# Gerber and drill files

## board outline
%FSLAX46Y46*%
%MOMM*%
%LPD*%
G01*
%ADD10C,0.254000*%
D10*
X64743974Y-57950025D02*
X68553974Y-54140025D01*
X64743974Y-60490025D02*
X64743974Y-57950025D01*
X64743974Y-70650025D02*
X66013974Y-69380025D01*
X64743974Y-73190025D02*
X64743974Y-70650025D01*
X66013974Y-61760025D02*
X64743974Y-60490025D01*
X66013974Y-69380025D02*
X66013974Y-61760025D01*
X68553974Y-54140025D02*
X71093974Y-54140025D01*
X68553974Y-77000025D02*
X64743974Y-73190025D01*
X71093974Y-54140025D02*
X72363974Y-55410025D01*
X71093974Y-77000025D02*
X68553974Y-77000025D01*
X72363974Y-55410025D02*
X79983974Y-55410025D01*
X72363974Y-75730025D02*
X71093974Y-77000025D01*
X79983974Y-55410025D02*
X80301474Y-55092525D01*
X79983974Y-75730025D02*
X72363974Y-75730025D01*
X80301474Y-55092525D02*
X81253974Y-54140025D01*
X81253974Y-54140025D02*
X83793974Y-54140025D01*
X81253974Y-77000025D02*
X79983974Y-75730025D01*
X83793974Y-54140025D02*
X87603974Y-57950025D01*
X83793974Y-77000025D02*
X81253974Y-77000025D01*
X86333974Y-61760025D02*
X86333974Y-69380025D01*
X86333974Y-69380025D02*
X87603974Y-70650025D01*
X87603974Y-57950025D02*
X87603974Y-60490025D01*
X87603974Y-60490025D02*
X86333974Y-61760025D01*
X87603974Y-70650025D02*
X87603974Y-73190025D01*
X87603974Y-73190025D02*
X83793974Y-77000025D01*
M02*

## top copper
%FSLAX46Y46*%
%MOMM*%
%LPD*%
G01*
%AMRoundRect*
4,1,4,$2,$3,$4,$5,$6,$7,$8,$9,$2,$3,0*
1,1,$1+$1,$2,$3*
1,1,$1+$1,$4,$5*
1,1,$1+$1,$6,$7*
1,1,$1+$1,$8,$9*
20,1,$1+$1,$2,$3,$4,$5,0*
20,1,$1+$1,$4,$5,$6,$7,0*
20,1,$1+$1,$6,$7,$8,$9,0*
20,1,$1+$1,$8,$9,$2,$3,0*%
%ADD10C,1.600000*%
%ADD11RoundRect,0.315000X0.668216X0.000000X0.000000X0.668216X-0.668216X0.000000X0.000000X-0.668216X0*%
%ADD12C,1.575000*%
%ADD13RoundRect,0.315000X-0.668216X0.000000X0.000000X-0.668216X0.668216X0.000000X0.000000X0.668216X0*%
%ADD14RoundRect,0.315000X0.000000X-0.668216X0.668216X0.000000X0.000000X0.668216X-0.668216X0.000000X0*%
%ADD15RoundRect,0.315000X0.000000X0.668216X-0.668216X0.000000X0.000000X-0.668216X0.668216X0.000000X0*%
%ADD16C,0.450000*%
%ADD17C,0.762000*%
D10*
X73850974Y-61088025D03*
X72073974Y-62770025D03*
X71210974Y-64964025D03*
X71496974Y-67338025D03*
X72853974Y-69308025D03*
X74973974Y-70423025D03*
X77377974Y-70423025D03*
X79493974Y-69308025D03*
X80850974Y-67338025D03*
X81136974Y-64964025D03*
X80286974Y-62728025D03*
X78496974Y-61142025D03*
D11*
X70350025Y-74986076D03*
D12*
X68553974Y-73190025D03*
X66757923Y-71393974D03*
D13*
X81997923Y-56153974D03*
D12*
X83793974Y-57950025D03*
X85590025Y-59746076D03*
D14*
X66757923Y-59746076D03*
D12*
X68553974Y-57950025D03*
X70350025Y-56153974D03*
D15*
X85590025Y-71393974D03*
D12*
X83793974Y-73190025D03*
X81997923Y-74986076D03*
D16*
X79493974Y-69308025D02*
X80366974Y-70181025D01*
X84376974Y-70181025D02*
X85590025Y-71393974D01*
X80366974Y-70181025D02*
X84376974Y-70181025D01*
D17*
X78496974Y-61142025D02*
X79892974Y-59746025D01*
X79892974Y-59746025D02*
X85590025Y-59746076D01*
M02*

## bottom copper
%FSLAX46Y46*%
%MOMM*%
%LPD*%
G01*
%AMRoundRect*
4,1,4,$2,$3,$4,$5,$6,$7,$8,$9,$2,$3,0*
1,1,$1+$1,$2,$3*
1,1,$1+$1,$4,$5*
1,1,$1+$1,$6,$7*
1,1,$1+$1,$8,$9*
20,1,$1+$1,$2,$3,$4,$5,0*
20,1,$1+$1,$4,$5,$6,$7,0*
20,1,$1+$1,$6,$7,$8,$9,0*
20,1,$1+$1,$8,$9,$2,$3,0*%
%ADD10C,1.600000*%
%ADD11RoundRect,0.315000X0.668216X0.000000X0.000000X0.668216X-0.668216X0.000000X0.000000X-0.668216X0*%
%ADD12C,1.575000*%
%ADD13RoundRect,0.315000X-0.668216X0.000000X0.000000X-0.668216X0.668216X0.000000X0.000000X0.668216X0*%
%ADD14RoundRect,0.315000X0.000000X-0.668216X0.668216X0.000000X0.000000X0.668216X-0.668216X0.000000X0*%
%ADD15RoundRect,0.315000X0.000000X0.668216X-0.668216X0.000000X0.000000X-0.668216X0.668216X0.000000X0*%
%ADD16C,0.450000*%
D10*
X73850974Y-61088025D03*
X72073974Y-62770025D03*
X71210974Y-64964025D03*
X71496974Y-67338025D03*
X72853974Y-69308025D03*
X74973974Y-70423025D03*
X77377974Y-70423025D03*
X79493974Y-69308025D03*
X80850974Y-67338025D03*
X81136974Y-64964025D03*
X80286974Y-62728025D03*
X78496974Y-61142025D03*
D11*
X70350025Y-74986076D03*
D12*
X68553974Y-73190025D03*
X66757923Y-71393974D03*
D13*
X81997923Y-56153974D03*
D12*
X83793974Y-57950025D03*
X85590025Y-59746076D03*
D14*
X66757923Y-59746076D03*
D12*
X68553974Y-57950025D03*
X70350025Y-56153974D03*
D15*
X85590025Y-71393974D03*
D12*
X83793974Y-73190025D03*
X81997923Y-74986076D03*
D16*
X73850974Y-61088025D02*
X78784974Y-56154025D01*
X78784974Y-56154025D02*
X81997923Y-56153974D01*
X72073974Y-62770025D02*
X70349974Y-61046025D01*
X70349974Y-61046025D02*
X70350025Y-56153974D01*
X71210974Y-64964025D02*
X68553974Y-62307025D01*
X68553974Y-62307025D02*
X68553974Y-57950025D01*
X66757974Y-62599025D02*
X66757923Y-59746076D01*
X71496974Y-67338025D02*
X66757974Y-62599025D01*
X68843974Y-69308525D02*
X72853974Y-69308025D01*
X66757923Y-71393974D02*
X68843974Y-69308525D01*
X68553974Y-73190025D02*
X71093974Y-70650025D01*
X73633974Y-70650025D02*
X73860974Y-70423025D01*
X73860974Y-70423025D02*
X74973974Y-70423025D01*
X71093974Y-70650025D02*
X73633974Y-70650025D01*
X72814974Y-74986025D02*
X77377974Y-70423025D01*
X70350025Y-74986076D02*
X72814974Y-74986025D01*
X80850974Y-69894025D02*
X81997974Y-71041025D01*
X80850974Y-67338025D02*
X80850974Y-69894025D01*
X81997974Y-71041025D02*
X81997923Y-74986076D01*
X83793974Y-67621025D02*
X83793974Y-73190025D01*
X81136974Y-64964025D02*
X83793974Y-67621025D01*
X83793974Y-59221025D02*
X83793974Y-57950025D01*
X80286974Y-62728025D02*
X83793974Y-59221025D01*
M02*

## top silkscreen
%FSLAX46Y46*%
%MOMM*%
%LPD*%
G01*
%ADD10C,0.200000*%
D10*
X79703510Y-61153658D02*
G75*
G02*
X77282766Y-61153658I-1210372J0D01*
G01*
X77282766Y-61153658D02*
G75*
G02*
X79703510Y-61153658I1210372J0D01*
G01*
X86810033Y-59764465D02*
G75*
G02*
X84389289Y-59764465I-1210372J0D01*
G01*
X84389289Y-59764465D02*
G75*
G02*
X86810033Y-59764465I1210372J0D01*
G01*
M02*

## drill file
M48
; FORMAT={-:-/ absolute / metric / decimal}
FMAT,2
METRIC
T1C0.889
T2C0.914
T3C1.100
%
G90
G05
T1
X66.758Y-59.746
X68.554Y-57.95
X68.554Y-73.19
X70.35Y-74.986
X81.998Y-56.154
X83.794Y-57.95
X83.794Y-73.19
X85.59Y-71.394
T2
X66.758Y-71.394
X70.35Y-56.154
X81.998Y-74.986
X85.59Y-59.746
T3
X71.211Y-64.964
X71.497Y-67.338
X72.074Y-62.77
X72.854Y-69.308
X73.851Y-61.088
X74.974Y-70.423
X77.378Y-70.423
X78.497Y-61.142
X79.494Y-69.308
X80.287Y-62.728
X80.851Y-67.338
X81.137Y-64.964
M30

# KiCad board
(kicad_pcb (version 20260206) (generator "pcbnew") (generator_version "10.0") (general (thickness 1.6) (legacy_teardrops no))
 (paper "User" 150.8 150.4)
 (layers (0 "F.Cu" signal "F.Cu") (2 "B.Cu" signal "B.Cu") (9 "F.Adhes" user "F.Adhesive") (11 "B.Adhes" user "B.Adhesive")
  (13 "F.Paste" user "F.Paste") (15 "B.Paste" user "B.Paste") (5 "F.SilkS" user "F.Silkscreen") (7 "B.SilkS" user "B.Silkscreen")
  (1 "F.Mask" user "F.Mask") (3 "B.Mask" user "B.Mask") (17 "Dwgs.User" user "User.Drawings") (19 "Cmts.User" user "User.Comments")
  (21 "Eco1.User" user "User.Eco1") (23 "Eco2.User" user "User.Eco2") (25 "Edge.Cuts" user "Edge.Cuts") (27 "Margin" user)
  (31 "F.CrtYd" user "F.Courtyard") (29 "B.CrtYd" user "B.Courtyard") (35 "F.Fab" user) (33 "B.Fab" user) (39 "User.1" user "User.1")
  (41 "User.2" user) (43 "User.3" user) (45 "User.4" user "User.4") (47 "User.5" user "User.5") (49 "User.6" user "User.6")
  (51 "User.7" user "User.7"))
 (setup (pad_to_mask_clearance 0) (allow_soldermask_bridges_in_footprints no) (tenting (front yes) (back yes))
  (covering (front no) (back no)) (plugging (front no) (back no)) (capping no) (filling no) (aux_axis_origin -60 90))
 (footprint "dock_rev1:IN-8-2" (layer "F.Cu") (at 76.173974 65.570025)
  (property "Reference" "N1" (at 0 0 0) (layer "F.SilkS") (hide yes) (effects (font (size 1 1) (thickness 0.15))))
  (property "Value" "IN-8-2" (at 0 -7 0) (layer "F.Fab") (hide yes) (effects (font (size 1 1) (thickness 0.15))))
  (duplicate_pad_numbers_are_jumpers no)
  (pad "2" thru_hole circle (at -2.323 -4.482) (size 1.6 1.6) (drill 1.1) (layers "*.Cu" "*.Mask") (remove_unused_layers no) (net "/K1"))
  (pad "3" thru_hole circle (at -4.1 -2.8) (size 1.6 1.6) (drill 1.1) (layers "*.Cu" "*.Mask") (remove_unused_layers no) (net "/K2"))
  (pad "4" thru_hole circle (at -4.963 -0.606) (size 1.6 1.6) (drill 1.1) (layers "*.Cu" "*.Mask") (remove_unused_layers no) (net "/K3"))
  (pad "5" thru_hole circle (at -4.677 1.768) (size 1.6 1.6) (drill 1.1) (layers "*.Cu" "*.Mask") (remove_unused_layers no) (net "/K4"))
  (pad "6" thru_hole circle (at -3.32 3.738) (size 1.6 1.6) (drill 1.1) (layers "*.Cu" "*.Mask") (remove_unused_layers no) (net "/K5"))
  (pad "7" thru_hole circle (at -1.2 4.853) (size 1.6 1.6) (drill 1.1) (layers "*.Cu" "*.Mask") (remove_unused_layers no) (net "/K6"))
  (pad "8" thru_hole circle (at 1.204 4.853) (size 1.6 1.6) (drill 1.1) (layers "*.Cu" "*.Mask") (remove_unused_layers no) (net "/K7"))
  (pad "9" thru_hole circle (at 3.32 3.738) (size 1.6 1.6) (drill 1.1) (layers "*.Cu" "*.Mask") (remove_unused_layers no) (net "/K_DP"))
  (pad "10" thru_hole circle (at 4.677 1.768) (size 1.6 1.6) (drill 1.1) (layers "*.Cu" "*.Mask") (remove_unused_layers no) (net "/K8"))
  (pad "11" thru_hole circle (at 4.963 -0.606) (size 1.6 1.6) (drill 1.1) (layers "*.Cu" "*.Mask") (remove_unused_layers no) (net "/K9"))
  (pad "12" thru_hole circle (at 4.113 -2.842) (size 1.6 1.6) (drill 1.1) (layers "*.Cu" "*.Mask") (remove_unused_layers no) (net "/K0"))
  (pad "13" thru_hole circle (at 2.323 -4.428) (size 1.6 1.6) (drill 1.1) (layers "*.Cu" "*.Mask") (remove_unused_layers no) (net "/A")))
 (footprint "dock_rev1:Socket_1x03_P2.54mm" (layer "B.Cu") (at 68.553974 73.190025 135)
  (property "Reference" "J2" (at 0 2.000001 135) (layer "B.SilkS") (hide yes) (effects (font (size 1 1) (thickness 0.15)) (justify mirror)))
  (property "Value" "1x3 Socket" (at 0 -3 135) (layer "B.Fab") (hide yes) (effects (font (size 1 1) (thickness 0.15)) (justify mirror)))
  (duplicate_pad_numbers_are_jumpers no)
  (pad "1" thru_hole roundrect (at -2.54 0 135) (size 1.575 1.575) (drill 0.889) (layers "*.Cu" "*.Mask") (remove_unused_layers no)
   (roundrect_rratio 0.2) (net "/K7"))
  (pad "2" thru_hole circle (at 0 0 135) (size 1.575 1.575) (drill 0.889) (layers "*.Cu" "*.Mask") (remove_unused_layers no) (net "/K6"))
  (pad "3" thru_hole circle (at 2.54 0 135) (size 1.575 1.575) (drill 0.9145) (layers "*.Cu" "*.Mask") (remove_unused_layers no) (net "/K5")))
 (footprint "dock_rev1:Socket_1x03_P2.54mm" (layer "B.Cu") (at 83.793974 57.950025 -45)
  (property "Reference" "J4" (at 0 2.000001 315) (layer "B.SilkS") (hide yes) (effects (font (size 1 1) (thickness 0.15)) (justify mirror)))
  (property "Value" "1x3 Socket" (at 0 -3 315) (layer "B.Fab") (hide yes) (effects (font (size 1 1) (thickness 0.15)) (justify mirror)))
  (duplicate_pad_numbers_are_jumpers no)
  (pad "1" thru_hole roundrect (at -2.54 0 315) (size 1.575 1.575) (drill 0.889) (layers "*.Cu" "*.Mask") (remove_unused_layers no)
   (roundrect_rratio 0.2) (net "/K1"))
  (pad "2" thru_hole circle (at 0 0 315) (size 1.575 1.575) (drill 0.889) (layers "*.Cu" "*.Mask") (remove_unused_layers no) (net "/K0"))
  (pad "3" thru_hole circle (at 2.54 0 315) (size 1.575 1.575) (drill 0.9145) (layers "*.Cu" "*.Mask") (remove_unused_layers no) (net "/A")))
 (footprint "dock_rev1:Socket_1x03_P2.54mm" (layer "B.Cu") (at 68.553974 57.950025 45)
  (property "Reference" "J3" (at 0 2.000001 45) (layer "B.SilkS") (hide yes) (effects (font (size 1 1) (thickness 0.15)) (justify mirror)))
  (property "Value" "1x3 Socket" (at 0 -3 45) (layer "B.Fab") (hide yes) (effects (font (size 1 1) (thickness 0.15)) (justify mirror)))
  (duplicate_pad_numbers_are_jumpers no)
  (pad "1" thru_hole roundrect (at -2.54 0 45) (size 1.575 1.575) (drill 0.889) (layers "*.Cu" "*.Mask") (remove_unused_layers no)
   (roundrect_rratio 0.2) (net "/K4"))
  (pad "2" thru_hole circle (at 0 0 45) (size 1.575 1.575) (drill 0.889) (layers "*.Cu" "*.Mask") (remove_unused_layers no) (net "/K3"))
  (pad "3" thru_hole circle (at 2.54 0 45) (size 1.575 1.575) (drill 0.9145) (layers "*.Cu" "*.Mask") (remove_unused_layers no) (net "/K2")))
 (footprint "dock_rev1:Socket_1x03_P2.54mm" (layer "B.Cu") (at 83.793974 73.190025 -135)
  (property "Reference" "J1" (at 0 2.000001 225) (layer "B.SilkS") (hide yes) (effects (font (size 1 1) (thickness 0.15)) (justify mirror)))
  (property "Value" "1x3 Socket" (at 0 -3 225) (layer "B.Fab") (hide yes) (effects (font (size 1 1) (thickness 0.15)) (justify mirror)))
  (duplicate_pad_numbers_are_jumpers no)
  (pad "1" thru_hole roundrect (at -2.54 0 225) (size 1.575 1.575) (drill 0.889) (layers "*.Cu" "*.Mask") (remove_unused_layers no)
   (roundrect_rratio 0.2) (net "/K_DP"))
  (pad "2" thru_hole circle (at 0 0 225) (size 1.575 1.575) (drill 0.889) (layers "*.Cu" "*.Mask") (remove_unused_layers no) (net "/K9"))
  (pad "3" thru_hole circle (at 2.54 0 225) (size 1.575 1.575) (drill 0.9145) (layers "*.Cu" "*.Mask") (remove_unused_layers no) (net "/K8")))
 (gr_circle (center 78.493138 61.153658) (end 79.243138 62.103658) (stroke (width 0.2) (type default)) (fill no) (layer "F.SilkS"))
 (gr_circle (center 85.599661 59.764465) (end 86.349661 60.714465) (stroke (width 0.2) (type default)) (fill no) (layer "F.SilkS"))
 (gr_line (start 64.743974 57.950025) (end 68.553974 54.140025) (stroke (width 0.254) (type default)) (layer "Edge.Cuts"))
 (gr_line (start 64.743974 60.490025) (end 64.743974 57.950025) (stroke (width 0.254) (type default)) (layer "Edge.Cuts"))
 (gr_line (start 64.743974 70.650025) (end 66.013974 69.380025) (stroke (width 0.254) (type default)) (layer "Edge.Cuts"))
 (gr_line (start 64.743974 73.190025) (end 64.743974 70.650025) (stroke (width 0.254) (type default)) (layer "Edge.Cuts"))
 (gr_line (start 66.013974 61.760025) (end 64.743974 60.490025) (stroke (width 0.254) (type default)) (layer "Edge.Cuts"))
 (gr_line (start 66.013974 69.380025) (end 66.013974 61.760025) (stroke (width 0.254) (type default)) (layer "Edge.Cuts"))
 (gr_line (start 68.553974 54.140025) (end 71.093974 54.140025) (stroke (width 0.254) (type default)) (layer "Edge.Cuts"))
 (gr_line (start 68.553974 77.000025) (end 64.743974 73.190025) (stroke (width 0.254) (type default)) (layer "Edge.Cuts"))
 (gr_line (start 71.093974 54.140025) (end 72.363974 55.410025) (stroke (width 0.254) (type default)) (layer "Edge.Cuts"))
 (gr_line (start 71.093974 77.000025) (end 68.553974 77.000025) (stroke (width 0.254) (type default)) (layer "Edge.Cuts"))
 (gr_line (start 72.363974 55.410025) (end 79.983974 55.410025) (stroke (width 0.254) (type default)) (layer "Edge.Cuts"))
 (gr_line (start 72.363974 75.730025) (end 71.093974 77.000025) (stroke (width 0.254) (type default)) (layer "Edge.Cuts"))
 (gr_line (start 79.983974 55.410025) (end 80.301474 55.092525) (stroke (width 0.254) (type default)) (layer "Edge.Cuts"))
 (gr_line (start 79.983974 75.730025) (end 72.363974 75.730025) (stroke (width 0.254) (type default)) (layer "Edge.Cuts"))
 (gr_line (start 80.301474 55.092525) (end 81.253974 54.140025) (stroke (width 0.254) (type default)) (layer "Edge.Cuts"))
 (gr_line (start 81.253974 54.140025) (end 83.793974 54.140025) (stroke (width 0.254) (type default)) (layer "Edge.Cuts"))
 (gr_line (start 81.253974 77.000025) (end 79.983974 75.730025) (stroke (width 0.254) (type default)) (layer "Edge.Cuts"))
 (gr_line (start 83.793974 54.140025) (end 87.603974 57.950025) (stroke (width 0.254) (type default)) (layer "Edge.Cuts"))
 (gr_line (start 83.793974 77.000025) (end 81.253974 77.000025) (stroke (width 0.254) (type default)) (layer "Edge.Cuts"))
 (gr_line (start 86.333974 61.760025) (end 86.333974 69.380025) (stroke (width 0.254) (type default)) (layer "Edge.Cuts"))
 (gr_line (start 86.333974 69.380025) (end 87.603974 70.650025) (stroke (width 0.254) (type default)) (layer "Edge.Cuts"))
 (gr_line (start 87.603974 57.950025) (end 87.603974 60.490025) (stroke (width 0.254) (type default)) (layer "Edge.Cuts"))
 (gr_line (start 87.603974 60.490025) (end 86.333974 61.760025) (stroke (width 0.254) (type default)) (layer "Edge.Cuts"))
 (gr_line (start 87.603974 70.650025) (end 87.603974 73.190025) (stroke (width 0.254) (type default)) (layer "Edge.Cuts"))
 (gr_line (start 87.603974 73.190025) (end 83.793974 77.000025) (stroke (width 0.254) (type default)) (layer "Edge.Cuts"))
 (segment (start 73.850974 61.088025) (end 78.784974 56.154025) (width 0.45) (layer "B.Cu") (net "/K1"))
 (segment (start 78.784974 56.154025) (end 81.997923 56.153974) (width 0.45) (layer "B.Cu") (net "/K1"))
 (segment (start 72.073974 62.770025) (end 70.349974 61.046025) (width 0.45) (layer "B.Cu") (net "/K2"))
 (segment (start 70.349974 61.046025) (end 70.350025 56.153974) (width 0.45) (layer "B.Cu") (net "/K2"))
 (segment (start 71.210974 64.964025) (end 68.553974 62.307025) (width 0.45) (layer "B.Cu") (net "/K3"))
 (segment (start 68.553974 62.307025) (end 68.553974 57.950025) (width 0.45) (layer "B.Cu") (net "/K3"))
 (segment (start 66.757974 62.599025) (end 66.757923 59.746076) (width 0.45) (layer "B.Cu") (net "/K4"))
 (segment (start 71.496974 67.338025) (end 66.757974 62.599025) (width 0.45) (layer "B.Cu") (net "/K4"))
 (segment (start 68.843974 69.308525) (end 72.853974 69.308025) (width 0.45) (layer "B.Cu") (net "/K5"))
 (segment (start 66.757923 71.393974) (end 68.843974 69.308525) (width 0.45) (layer "B.Cu") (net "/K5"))
 (segment (start 68.553974 73.190025) (end 71.093974 70.650025) (width 0.45) (layer "B.Cu") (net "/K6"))
 (segment (start 73.633974 70.650025) (end 73.860974 70.423025) (width 0.45) (layer "B.Cu") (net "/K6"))
 (segment (start 73.860974 70.423025) (end 74.973974 70.423025) (width 0.45) (layer "B.Cu") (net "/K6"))
 (segment (start 71.093974 70.650025) (end 73.633974 70.650025) (width 0.45) (layer "B.Cu") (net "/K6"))
 (segment (start 72.814974 74.986025) (end 77.377974 70.423025) (width 0.45) (layer "B.Cu") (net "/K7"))
 (segment (start 70.350025 74.986076) (end 72.814974 74.986025) (width 0.45) (layer "B.Cu") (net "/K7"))
 (segment (start 79.493974 69.308025) (end 80.366974 70.181025) (width 0.45) (layer "F.Cu") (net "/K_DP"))
 (segment (start 84.376974 70.181025) (end 85.590025 71.393974) (width 0.45) (layer "F.Cu") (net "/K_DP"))
 (segment (start 80.366974 70.181025) (end 84.376974 70.181025) (width 0.45) (layer "F.Cu") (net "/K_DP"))
 (segment (start 80.850974 69.894025) (end 81.997974 71.041025) (width 0.45) (layer "B.Cu") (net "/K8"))
 (segment (start 80.850974 67.338025) (end 80.850974 69.894025) (width 0.45) (layer "B.Cu") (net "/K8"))
 (segment (start 81.997974 71.041025) (end 81.997923 74.986076) (width 0.45) (layer "B.Cu") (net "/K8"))
 (segment (start 83.793974 67.621025) (end 83.793974 73.190025) (width 0.45) (layer "B.Cu") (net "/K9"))
 (segment (start 81.136974 64.964025) (end 83.793974 67.621025) (width 0.45) (layer "B.Cu") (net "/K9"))
 (segment (start 83.793974 59.221025) (end 83.793974 57.950025) (width 0.45) (layer "B.Cu") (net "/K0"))
 (segment (start 80.286974 62.728025) (end 83.793974 59.221025) (width 0.45) (layer "B.Cu") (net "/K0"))
 (segment (start 78.496974 61.142025) (end 79.892974 59.746025) (width 0.762) (layer "F.Cu") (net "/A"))
 (segment (start 79.892974 59.746025) (end 85.590025 59.746076) (width 0.762) (layer "F.Cu") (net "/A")))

